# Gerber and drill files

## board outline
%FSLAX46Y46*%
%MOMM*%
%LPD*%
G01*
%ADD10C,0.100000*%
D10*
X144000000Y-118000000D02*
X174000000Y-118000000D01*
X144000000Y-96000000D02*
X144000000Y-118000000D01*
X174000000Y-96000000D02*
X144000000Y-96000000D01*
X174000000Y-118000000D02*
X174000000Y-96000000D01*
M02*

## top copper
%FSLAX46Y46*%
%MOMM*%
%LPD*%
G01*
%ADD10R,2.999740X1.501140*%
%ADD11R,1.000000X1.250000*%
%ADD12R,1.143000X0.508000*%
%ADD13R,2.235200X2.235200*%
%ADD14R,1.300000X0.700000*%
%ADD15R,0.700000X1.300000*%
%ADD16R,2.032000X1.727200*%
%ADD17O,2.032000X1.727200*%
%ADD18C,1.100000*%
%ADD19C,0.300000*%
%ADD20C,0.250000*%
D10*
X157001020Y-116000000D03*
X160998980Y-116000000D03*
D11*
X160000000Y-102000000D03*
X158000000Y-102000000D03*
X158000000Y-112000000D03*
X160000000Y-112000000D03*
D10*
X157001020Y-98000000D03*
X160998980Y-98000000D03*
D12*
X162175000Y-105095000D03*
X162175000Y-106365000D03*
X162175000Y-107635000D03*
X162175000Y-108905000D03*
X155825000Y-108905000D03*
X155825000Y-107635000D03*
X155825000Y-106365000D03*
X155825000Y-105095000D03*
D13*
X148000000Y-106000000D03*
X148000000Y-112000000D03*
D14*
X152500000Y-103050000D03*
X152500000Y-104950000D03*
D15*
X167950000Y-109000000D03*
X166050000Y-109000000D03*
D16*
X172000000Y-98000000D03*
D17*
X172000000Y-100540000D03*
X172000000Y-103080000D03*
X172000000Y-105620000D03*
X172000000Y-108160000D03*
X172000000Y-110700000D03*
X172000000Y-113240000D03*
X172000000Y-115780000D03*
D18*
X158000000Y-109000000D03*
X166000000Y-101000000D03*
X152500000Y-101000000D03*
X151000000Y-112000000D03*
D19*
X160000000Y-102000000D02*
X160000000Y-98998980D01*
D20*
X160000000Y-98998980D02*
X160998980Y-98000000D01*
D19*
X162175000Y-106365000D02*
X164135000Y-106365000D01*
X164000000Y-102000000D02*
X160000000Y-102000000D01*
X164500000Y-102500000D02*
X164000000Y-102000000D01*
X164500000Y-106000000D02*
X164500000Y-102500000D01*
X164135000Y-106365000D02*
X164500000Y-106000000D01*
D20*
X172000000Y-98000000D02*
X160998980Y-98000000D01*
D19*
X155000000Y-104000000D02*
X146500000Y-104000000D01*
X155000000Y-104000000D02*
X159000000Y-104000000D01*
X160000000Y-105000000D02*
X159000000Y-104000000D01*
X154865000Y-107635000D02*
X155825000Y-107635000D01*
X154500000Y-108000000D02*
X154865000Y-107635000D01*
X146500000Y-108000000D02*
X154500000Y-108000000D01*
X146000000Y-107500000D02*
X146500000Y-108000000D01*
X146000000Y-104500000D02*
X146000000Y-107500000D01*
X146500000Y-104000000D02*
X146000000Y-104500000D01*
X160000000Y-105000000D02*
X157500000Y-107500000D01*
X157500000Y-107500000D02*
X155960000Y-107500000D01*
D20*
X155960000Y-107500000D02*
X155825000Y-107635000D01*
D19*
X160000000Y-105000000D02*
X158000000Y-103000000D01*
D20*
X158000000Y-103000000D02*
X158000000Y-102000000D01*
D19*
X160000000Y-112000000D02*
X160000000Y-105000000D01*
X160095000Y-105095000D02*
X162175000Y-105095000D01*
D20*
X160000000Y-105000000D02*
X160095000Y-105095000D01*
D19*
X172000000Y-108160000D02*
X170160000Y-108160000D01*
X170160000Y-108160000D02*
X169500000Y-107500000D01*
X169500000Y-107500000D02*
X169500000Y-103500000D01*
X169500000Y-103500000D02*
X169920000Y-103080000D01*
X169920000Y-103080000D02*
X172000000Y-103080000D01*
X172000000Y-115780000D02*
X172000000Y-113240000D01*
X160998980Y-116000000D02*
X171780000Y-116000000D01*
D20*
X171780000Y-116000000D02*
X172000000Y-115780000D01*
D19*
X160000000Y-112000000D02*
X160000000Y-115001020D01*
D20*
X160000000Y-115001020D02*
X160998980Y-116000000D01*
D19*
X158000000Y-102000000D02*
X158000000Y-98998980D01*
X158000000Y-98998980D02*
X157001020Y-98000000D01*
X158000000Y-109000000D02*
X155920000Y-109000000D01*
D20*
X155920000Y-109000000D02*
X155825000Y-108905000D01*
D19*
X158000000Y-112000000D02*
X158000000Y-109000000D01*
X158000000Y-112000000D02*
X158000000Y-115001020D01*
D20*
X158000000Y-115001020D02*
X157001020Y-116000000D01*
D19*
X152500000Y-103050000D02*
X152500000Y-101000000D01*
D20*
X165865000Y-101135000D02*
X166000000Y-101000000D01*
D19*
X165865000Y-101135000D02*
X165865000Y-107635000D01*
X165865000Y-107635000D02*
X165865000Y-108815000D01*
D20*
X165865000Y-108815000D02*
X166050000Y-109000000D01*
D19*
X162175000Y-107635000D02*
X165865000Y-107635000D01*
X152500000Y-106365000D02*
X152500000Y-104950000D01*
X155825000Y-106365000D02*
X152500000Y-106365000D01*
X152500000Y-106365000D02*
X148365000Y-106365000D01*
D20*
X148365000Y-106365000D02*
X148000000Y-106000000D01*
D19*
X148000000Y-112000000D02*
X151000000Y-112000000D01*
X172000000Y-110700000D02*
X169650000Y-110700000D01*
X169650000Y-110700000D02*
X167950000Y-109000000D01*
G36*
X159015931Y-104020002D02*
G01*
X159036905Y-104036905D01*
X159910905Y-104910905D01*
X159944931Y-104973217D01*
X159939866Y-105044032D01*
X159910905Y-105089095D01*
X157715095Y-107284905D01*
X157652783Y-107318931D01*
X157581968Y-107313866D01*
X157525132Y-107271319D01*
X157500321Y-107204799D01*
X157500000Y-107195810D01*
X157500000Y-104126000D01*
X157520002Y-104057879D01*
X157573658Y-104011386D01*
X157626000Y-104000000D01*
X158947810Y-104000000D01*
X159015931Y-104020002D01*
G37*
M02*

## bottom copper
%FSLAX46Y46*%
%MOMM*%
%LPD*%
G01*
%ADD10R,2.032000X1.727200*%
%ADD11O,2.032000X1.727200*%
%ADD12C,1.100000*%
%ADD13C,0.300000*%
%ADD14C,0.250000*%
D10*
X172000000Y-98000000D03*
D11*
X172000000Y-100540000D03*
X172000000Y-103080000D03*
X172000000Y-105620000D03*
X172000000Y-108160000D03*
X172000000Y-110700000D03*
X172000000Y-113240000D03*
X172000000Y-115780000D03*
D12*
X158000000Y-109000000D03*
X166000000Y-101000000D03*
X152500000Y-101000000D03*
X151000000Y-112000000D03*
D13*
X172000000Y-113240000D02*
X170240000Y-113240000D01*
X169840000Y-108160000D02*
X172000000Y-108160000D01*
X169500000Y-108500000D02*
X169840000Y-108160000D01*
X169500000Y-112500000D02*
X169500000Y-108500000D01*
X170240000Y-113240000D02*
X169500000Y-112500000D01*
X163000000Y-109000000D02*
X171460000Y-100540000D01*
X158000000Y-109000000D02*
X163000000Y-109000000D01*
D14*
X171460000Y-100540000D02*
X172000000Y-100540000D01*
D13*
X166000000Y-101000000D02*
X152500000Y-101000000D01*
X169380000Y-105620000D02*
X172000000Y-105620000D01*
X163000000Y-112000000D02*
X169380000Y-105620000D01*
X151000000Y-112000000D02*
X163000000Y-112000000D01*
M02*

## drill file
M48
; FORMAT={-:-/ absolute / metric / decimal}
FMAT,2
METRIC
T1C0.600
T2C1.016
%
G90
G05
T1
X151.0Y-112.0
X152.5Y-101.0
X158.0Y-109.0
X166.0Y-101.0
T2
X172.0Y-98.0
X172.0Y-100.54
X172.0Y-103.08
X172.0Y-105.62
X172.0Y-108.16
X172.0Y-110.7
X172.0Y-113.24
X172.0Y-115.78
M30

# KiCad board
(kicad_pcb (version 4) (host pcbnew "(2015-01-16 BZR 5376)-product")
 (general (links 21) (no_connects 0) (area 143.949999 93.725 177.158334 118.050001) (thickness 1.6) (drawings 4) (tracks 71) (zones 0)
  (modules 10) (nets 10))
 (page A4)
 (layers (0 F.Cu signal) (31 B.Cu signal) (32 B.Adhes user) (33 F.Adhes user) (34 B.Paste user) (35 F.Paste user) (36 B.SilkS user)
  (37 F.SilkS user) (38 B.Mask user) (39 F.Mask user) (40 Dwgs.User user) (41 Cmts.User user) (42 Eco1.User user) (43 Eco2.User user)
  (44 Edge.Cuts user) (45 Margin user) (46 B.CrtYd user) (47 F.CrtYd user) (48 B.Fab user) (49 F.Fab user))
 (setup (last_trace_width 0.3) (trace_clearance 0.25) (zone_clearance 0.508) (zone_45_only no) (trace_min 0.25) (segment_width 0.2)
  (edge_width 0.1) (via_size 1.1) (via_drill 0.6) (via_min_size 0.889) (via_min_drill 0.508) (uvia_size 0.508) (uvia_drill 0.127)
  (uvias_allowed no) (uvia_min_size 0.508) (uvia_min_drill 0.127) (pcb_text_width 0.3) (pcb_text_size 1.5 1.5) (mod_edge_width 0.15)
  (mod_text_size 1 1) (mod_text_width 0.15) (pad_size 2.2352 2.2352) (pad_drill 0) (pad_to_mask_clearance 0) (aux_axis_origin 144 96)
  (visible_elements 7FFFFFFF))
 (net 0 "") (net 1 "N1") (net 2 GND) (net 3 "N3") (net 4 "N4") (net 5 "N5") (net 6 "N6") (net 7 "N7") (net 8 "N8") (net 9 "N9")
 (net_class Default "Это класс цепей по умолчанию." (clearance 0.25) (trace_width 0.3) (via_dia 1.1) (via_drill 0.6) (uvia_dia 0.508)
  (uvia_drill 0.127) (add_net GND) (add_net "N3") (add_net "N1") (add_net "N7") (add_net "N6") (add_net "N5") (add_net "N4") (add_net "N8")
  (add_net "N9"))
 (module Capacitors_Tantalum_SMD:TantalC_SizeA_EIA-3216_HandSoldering (layer F.Cu) (at 159 116 180)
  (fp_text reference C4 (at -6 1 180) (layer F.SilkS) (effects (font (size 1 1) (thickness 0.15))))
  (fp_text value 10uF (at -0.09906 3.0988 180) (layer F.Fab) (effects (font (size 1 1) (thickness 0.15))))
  (pad 2 smd rect (at 1.99898 0 180) (size 2.99974 1.50114) (layers F.Cu F.Paste F.Mask) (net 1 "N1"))
  (pad 1 smd rect (at -1.99898 0 180) (size 2.99974 1.50114) (layers F.Cu F.Paste F.Mask) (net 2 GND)))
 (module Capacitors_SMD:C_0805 (layer F.Cu) (at 159 102 180)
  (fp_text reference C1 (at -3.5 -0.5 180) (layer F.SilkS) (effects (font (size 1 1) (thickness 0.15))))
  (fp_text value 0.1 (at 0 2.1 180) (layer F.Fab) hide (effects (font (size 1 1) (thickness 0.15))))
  (pad 1 smd rect (at -1 0 180) (size 1 1.25) (layers F.Cu F.Paste F.Mask) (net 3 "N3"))
  (pad 2 smd rect (at 1 0 180) (size 1 1.25) (layers F.Cu F.Paste F.Mask) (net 2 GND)))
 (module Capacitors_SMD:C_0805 (layer F.Cu) (at 159 112)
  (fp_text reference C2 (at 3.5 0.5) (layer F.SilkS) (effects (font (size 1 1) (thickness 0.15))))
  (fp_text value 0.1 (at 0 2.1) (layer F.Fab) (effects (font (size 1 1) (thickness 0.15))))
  (pad 1 smd rect (at -1 0) (size 1 1.25) (layers F.Cu F.Paste F.Mask) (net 1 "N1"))
  (pad 2 smd rect (at 1 0) (size 1 1.25) (layers F.Cu F.Paste F.Mask) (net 2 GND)))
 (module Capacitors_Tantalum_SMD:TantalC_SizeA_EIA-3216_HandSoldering (layer F.Cu) (at 159 98 180)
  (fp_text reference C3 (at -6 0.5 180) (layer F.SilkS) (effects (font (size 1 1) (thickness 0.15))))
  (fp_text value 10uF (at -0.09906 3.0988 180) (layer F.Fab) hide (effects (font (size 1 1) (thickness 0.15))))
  (pad 2 smd rect (at 1.99898 0 180) (size 2.99974 1.50114) (layers F.Cu F.Paste F.Mask) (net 2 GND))
  (pad 1 smd rect (at -1.99898 0 180) (size 2.99974 1.50114) (layers F.Cu F.Paste F.Mask) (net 3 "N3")))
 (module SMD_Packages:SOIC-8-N (layer F.Cu) (at 159 107 270)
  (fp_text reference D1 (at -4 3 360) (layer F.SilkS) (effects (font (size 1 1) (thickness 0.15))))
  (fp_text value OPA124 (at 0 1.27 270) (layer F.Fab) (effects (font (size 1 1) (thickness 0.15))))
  (pad 8 smd rect (at -1.905 -3.175 270) (size 0.508 1.143) (layers F.Cu F.Paste F.Mask) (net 2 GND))
  (pad 7 smd rect (at -0.635 -3.175 270) (size 0.508 1.143) (layers F.Cu F.Paste F.Mask) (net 3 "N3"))
  (pad 6 smd rect (at 0.635 -3.175 270) (size 0.508 1.143) (layers F.Cu F.Paste F.Mask) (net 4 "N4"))
  (pad 5 smd rect (at 1.905 -3.175 270) (size 0.508 1.143) (layers F.Cu F.Paste F.Mask) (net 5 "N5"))
  (pad 4 smd rect (at 1.905 3.175 270) (size 0.508 1.143) (layers F.Cu F.Paste F.Mask) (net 1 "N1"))
  (pad 3 smd rect (at 0.635 3.175 270) (size 0.508 1.143) (layers F.Cu F.Paste F.Mask) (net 2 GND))
  (pad 2 smd rect (at -0.635 3.175 270) (size 0.508 1.143) (layers F.Cu F.Paste F.Mask) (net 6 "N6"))
  (pad 1 smd rect (at -1.905 3.175 270) (size 0.508 1.143) (layers F.Cu F.Paste F.Mask) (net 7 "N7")))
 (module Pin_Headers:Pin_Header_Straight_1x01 (layer F.Cu) (at 148 106)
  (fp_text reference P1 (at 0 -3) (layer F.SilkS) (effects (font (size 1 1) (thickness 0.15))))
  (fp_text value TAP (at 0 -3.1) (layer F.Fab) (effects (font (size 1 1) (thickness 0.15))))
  (pad 1 smd rect (at 0 0) (size 2.2352 2.2352) (layers F.Cu F.Paste F.Mask) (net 6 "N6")))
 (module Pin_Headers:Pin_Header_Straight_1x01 (layer F.Cu) (at 148 112)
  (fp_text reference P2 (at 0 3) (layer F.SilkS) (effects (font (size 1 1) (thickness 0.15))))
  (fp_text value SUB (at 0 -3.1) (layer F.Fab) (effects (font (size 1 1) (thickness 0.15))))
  (pad 1 smd rect (at 0 0) (size 2.2352 2.2352) (layers F.Cu F.Paste F.Mask) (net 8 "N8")))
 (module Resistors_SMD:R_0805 (layer F.Cu) (at 152.5 104 270)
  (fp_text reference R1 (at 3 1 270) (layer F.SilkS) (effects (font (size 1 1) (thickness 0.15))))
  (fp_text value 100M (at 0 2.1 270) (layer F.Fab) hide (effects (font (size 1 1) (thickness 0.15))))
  (pad 1 smd rect (at -0.95 0 270) (size 0.7 1.3) (layers F.Cu F.Paste F.Mask) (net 4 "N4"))
  (pad 2 smd rect (at 0.95 0 270) (size 0.7 1.3) (layers F.Cu F.Paste F.Mask) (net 6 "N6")))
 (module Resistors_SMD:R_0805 (layer F.Cu) (at 167 109 180)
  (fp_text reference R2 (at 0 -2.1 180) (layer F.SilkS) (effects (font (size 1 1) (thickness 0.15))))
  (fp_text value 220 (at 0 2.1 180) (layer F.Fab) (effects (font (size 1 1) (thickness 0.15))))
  (pad 1 smd rect (at -0.95 0 180) (size 0.7 1.3) (layers F.Cu F.Paste F.Mask) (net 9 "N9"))
  (pad 2 smd rect (at 0.95 0 180) (size 0.7 1.3) (layers F.Cu F.Paste F.Mask) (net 4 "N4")))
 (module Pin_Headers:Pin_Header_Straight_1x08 (layer F.Cu) (at 172 98)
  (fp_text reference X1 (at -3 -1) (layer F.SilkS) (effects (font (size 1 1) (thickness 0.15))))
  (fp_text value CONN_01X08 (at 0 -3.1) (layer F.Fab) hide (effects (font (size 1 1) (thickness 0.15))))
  (pad 1 thru_hole rect (at 0 0) (size 2.032 1.7272) (drill 1.016) (layers *.Cu *.Mask F.SilkS) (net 3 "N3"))
  (pad 2 thru_hole oval (at 0 2.54) (size 2.032 1.7272) (drill 1.016) (layers *.Cu *.Mask F.SilkS) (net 1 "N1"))
  (pad 3 thru_hole oval (at 0 5.08) (size 2.032 1.7272) (drill 1.016) (layers *.Cu *.Mask F.SilkS) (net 2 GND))
  (pad 4 thru_hole oval (at 0 7.62) (size 2.032 1.7272) (drill 1.016) (layers *.Cu *.Mask F.SilkS) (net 8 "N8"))
  (pad 5 thru_hole oval (at 0 10.16) (size 2.032 1.7272) (drill 1.016) (layers *.Cu *.Mask F.SilkS) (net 2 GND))
  (pad 6 thru_hole oval (at 0 12.7) (size 2.032 1.7272) (drill 1.016) (layers *.Cu *.Mask F.SilkS) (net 9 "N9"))
  (pad 7 thru_hole oval (at 0 15.24) (size 2.032 1.7272) (drill 1.016) (layers *.Cu *.Mask F.SilkS) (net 2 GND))
  (pad 8 thru_hole oval (at 0 17.78) (size 2.032 1.7272) (drill 1.016) (layers *.Cu *.Mask F.SilkS) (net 2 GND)))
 (gr_line (start 144 118) (end 174 118) (angle 90) (layer Edge.Cuts) (width 0.1))
 (gr_line (start 144 96) (end 144 118) (angle 90) (layer Edge.Cuts) (width 0.1))
 (gr_line (start 174 96) (end 144 96) (angle 90) (layer Edge.Cuts) (width 0.1))
 (gr_line (start 174 118) (end 174 96) (angle 90) (layer Edge.Cuts) (width 0.1))
 (segment (start 160 102) (end 160 98.99898) (width 0.3) (layer F.Cu) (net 3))
 (segment (start 160 98.99898) (end 160.99898 98) (width 0.25) (layer F.Cu) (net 3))
 (segment (start 162.175 106.365) (end 164.135 106.365) (width 0.3) (layer F.Cu) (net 3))
 (segment (start 164 102) (end 160 102) (width 0.3) (layer F.Cu) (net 3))
 (segment (start 164.5 102.5) (end 164 102) (width 0.3) (layer F.Cu) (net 3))
 (segment (start 164.5 106) (end 164.5 102.5) (width 0.3) (layer F.Cu) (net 3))
 (segment (start 164.135 106.365) (end 164.5 106) (width 0.3) (layer F.Cu) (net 3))
 (segment (start 172 98) (end 160.99898 98) (width 0.25) (layer F.Cu) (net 3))
 (segment (start 155 104) (end 146.5 104) (width 0.3) (layer F.Cu) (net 2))
 (segment (start 155 104) (end 159 104) (width 0.3) (layer F.Cu) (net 2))
 (segment (start 160 105) (end 159 104) (width 0.3) (layer F.Cu) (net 2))
 (segment (start 154.865 107.635) (end 155.825 107.635) (width 0.3) (layer F.Cu) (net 2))
 (segment (start 154.5 108) (end 154.865 107.635) (width 0.3) (layer F.Cu) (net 2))
 (segment (start 146.5 108) (end 154.5 108) (width 0.3) (layer F.Cu) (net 2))
 (segment (start 146 107.5) (end 146.5 108) (width 0.3) (layer F.Cu) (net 2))
 (segment (start 146 104.5) (end 146 107.5) (width 0.3) (layer F.Cu) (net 2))
 (segment (start 146.5 104) (end 146 104.5) (width 0.3) (layer F.Cu) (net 2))
 (segment (start 160 105) (end 157.5 107.5) (width 0.3) (layer F.Cu) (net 2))
 (segment (start 157.5 107.5) (end 155.96 107.5) (width 0.3) (layer F.Cu) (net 2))
 (segment (start 155.96 107.5) (end 155.825 107.635) (width 0.25) (layer F.Cu) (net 2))
 (segment (start 160 105) (end 158 103) (width 0.3) (layer F.Cu) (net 2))
 (segment (start 158 103) (end 158 102) (width 0.25) (layer F.Cu) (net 2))
 (segment (start 160 112) (end 160 105) (width 0.3) (layer F.Cu) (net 2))
 (segment (start 160.095 105.095) (end 162.175 105.095) (width 0.3) (layer F.Cu) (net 2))
 (segment (start 160 105) (end 160.095 105.095) (width 0.25) (layer F.Cu) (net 2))
 (segment (start 172 113.24) (end 170.24 113.24) (width 0.3) (layer B.Cu) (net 2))
 (segment (start 169.84 108.16) (end 172 108.16) (width 0.3) (layer B.Cu) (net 2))
 (segment (start 169.5 108.5) (end 169.84 108.16) (width 0.3) (layer B.Cu) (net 2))
 (segment (start 169.5 112.5) (end 169.5 108.5) (width 0.3) (layer B.Cu) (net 2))
 (segment (start 170.24 113.24) (end 169.5 112.5) (width 0.3) (layer B.Cu) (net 2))
 (segment (start 172 108.16) (end 170.16 108.16) (width 0.3) (layer F.Cu) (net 2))
 (segment (start 170.16 108.16) (end 169.5 107.5) (width 0.3) (layer F.Cu) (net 2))
 (segment (start 169.5 107.5) (end 169.5 103.5) (width 0.3) (layer F.Cu) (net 2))
 (segment (start 169.5 103.5) (end 169.92 103.08) (width 0.3) (layer F.Cu) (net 2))
 (segment (start 169.92 103.08) (end 172 103.08) (width 0.3) (layer F.Cu) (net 2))
 (segment (start 172 115.78) (end 172 113.24) (width 0.3) (layer F.Cu) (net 2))
 (segment (start 160.99898 116) (end 171.78 116) (width 0.3) (layer F.Cu) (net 2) (status 10))
 (segment (start 171.78 116) (end 172 115.78) (width 0.25) (layer F.Cu) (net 2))
 (segment (start 160 112) (end 160 115.00102) (width 0.3) (layer F.Cu) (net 2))
 (segment (start 160 115.00102) (end 160.99898 116) (width 0.25) (layer F.Cu) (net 2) (status 20))
 (segment (start 158 102) (end 158 98.99898) (width 0.3) (layer F.Cu) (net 2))
 (segment (start 158 98.99898) (end 157.00102 98) (width 0.3) (layer F.Cu) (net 2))
 (segment (start 158 109) (end 155.92 109) (width 0.3) (layer F.Cu) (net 1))
 (segment (start 155.92 109) (end 155.825 108.905) (width 0.25) (layer F.Cu) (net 1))
 (segment (start 158 112) (end 158 109) (width 0.3) (layer F.Cu) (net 1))
 (segment (start 163 109) (end 171.46 100.54) (width 0.3) (layer B.Cu) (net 1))
 (segment (start 158 109) (end 163 109) (width 0.3) (layer B.Cu) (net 1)) (via (at 158 109) (size 1.1) (layers F.Cu B.Cu) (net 1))
 (segment (start 171.46 100.54) (end 172 100.54) (width 0.25) (layer B.Cu) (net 1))
 (segment (start 158 112) (end 158 115.00102) (width 0.3) (layer F.Cu) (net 1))
 (segment (start 158 115.00102) (end 157.00102 116) (width 0.25) (layer F.Cu) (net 1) (status 20))
 (segment (start 152.5 103.05) (end 152.5 101) (width 0.3) (layer F.Cu) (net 4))
 (segment (start 165.865 101.135) (end 166 101) (width 0.25) (layer F.Cu) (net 4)) (via (at 166 101) (size 1.1) (layers F.Cu B.Cu) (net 4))
 (segment (start 166 101) (end 152.5 101) (width 0.3) (layer B.Cu) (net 4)) (via (at 152.5 101) (size 1.1) (layers F.Cu B.Cu) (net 4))
 (segment (start 165.865 101.135) (end 165.865 107.635) (width 0.3) (layer F.Cu) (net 4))
 (segment (start 165.865 107.635) (end 165.865 108.815) (width 0.3) (layer F.Cu) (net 4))
 (segment (start 165.865 108.815) (end 166.05 109) (width 0.25) (layer F.Cu) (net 4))
 (segment (start 162.175 107.635) (end 165.865 107.635) (width 0.3) (layer F.Cu) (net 4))
 (segment (start 152.5 106.365) (end 152.5 104.95) (width 0.3) (layer F.Cu) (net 6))
 (segment (start 155.825 106.365) (end 152.5 106.365) (width 0.3) (layer F.Cu) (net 6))
 (segment (start 152.5 106.365) (end 148.365 106.365) (width 0.3) (layer F.Cu) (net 6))
 (segment (start 148.365 106.365) (end 148 106) (width 0.25) (layer F.Cu) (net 6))
 (segment (start 148 112) (end 151 112) (width 0.3) (layer F.Cu) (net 8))
 (segment (start 169.38 105.62) (end 172 105.62) (width 0.3) (layer B.Cu) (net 8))
 (segment (start 163 112) (end 169.38 105.62) (width 0.3) (layer B.Cu) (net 8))
 (segment (start 151 112) (end 163 112) (width 0.3) (layer B.Cu) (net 8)) (via (at 151 112) (size 1.1) (layers F.Cu B.Cu) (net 8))
 (segment (start 172 110.7) (end 169.65 110.7) (width 0.3) (layer F.Cu) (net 9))
 (segment (start 169.65 110.7) (end 167.95 109) (width 0.3) (layer F.Cu) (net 9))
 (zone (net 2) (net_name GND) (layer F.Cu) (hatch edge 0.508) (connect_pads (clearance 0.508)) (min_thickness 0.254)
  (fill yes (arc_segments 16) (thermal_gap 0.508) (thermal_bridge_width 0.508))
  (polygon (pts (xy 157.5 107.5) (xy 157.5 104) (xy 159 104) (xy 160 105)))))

